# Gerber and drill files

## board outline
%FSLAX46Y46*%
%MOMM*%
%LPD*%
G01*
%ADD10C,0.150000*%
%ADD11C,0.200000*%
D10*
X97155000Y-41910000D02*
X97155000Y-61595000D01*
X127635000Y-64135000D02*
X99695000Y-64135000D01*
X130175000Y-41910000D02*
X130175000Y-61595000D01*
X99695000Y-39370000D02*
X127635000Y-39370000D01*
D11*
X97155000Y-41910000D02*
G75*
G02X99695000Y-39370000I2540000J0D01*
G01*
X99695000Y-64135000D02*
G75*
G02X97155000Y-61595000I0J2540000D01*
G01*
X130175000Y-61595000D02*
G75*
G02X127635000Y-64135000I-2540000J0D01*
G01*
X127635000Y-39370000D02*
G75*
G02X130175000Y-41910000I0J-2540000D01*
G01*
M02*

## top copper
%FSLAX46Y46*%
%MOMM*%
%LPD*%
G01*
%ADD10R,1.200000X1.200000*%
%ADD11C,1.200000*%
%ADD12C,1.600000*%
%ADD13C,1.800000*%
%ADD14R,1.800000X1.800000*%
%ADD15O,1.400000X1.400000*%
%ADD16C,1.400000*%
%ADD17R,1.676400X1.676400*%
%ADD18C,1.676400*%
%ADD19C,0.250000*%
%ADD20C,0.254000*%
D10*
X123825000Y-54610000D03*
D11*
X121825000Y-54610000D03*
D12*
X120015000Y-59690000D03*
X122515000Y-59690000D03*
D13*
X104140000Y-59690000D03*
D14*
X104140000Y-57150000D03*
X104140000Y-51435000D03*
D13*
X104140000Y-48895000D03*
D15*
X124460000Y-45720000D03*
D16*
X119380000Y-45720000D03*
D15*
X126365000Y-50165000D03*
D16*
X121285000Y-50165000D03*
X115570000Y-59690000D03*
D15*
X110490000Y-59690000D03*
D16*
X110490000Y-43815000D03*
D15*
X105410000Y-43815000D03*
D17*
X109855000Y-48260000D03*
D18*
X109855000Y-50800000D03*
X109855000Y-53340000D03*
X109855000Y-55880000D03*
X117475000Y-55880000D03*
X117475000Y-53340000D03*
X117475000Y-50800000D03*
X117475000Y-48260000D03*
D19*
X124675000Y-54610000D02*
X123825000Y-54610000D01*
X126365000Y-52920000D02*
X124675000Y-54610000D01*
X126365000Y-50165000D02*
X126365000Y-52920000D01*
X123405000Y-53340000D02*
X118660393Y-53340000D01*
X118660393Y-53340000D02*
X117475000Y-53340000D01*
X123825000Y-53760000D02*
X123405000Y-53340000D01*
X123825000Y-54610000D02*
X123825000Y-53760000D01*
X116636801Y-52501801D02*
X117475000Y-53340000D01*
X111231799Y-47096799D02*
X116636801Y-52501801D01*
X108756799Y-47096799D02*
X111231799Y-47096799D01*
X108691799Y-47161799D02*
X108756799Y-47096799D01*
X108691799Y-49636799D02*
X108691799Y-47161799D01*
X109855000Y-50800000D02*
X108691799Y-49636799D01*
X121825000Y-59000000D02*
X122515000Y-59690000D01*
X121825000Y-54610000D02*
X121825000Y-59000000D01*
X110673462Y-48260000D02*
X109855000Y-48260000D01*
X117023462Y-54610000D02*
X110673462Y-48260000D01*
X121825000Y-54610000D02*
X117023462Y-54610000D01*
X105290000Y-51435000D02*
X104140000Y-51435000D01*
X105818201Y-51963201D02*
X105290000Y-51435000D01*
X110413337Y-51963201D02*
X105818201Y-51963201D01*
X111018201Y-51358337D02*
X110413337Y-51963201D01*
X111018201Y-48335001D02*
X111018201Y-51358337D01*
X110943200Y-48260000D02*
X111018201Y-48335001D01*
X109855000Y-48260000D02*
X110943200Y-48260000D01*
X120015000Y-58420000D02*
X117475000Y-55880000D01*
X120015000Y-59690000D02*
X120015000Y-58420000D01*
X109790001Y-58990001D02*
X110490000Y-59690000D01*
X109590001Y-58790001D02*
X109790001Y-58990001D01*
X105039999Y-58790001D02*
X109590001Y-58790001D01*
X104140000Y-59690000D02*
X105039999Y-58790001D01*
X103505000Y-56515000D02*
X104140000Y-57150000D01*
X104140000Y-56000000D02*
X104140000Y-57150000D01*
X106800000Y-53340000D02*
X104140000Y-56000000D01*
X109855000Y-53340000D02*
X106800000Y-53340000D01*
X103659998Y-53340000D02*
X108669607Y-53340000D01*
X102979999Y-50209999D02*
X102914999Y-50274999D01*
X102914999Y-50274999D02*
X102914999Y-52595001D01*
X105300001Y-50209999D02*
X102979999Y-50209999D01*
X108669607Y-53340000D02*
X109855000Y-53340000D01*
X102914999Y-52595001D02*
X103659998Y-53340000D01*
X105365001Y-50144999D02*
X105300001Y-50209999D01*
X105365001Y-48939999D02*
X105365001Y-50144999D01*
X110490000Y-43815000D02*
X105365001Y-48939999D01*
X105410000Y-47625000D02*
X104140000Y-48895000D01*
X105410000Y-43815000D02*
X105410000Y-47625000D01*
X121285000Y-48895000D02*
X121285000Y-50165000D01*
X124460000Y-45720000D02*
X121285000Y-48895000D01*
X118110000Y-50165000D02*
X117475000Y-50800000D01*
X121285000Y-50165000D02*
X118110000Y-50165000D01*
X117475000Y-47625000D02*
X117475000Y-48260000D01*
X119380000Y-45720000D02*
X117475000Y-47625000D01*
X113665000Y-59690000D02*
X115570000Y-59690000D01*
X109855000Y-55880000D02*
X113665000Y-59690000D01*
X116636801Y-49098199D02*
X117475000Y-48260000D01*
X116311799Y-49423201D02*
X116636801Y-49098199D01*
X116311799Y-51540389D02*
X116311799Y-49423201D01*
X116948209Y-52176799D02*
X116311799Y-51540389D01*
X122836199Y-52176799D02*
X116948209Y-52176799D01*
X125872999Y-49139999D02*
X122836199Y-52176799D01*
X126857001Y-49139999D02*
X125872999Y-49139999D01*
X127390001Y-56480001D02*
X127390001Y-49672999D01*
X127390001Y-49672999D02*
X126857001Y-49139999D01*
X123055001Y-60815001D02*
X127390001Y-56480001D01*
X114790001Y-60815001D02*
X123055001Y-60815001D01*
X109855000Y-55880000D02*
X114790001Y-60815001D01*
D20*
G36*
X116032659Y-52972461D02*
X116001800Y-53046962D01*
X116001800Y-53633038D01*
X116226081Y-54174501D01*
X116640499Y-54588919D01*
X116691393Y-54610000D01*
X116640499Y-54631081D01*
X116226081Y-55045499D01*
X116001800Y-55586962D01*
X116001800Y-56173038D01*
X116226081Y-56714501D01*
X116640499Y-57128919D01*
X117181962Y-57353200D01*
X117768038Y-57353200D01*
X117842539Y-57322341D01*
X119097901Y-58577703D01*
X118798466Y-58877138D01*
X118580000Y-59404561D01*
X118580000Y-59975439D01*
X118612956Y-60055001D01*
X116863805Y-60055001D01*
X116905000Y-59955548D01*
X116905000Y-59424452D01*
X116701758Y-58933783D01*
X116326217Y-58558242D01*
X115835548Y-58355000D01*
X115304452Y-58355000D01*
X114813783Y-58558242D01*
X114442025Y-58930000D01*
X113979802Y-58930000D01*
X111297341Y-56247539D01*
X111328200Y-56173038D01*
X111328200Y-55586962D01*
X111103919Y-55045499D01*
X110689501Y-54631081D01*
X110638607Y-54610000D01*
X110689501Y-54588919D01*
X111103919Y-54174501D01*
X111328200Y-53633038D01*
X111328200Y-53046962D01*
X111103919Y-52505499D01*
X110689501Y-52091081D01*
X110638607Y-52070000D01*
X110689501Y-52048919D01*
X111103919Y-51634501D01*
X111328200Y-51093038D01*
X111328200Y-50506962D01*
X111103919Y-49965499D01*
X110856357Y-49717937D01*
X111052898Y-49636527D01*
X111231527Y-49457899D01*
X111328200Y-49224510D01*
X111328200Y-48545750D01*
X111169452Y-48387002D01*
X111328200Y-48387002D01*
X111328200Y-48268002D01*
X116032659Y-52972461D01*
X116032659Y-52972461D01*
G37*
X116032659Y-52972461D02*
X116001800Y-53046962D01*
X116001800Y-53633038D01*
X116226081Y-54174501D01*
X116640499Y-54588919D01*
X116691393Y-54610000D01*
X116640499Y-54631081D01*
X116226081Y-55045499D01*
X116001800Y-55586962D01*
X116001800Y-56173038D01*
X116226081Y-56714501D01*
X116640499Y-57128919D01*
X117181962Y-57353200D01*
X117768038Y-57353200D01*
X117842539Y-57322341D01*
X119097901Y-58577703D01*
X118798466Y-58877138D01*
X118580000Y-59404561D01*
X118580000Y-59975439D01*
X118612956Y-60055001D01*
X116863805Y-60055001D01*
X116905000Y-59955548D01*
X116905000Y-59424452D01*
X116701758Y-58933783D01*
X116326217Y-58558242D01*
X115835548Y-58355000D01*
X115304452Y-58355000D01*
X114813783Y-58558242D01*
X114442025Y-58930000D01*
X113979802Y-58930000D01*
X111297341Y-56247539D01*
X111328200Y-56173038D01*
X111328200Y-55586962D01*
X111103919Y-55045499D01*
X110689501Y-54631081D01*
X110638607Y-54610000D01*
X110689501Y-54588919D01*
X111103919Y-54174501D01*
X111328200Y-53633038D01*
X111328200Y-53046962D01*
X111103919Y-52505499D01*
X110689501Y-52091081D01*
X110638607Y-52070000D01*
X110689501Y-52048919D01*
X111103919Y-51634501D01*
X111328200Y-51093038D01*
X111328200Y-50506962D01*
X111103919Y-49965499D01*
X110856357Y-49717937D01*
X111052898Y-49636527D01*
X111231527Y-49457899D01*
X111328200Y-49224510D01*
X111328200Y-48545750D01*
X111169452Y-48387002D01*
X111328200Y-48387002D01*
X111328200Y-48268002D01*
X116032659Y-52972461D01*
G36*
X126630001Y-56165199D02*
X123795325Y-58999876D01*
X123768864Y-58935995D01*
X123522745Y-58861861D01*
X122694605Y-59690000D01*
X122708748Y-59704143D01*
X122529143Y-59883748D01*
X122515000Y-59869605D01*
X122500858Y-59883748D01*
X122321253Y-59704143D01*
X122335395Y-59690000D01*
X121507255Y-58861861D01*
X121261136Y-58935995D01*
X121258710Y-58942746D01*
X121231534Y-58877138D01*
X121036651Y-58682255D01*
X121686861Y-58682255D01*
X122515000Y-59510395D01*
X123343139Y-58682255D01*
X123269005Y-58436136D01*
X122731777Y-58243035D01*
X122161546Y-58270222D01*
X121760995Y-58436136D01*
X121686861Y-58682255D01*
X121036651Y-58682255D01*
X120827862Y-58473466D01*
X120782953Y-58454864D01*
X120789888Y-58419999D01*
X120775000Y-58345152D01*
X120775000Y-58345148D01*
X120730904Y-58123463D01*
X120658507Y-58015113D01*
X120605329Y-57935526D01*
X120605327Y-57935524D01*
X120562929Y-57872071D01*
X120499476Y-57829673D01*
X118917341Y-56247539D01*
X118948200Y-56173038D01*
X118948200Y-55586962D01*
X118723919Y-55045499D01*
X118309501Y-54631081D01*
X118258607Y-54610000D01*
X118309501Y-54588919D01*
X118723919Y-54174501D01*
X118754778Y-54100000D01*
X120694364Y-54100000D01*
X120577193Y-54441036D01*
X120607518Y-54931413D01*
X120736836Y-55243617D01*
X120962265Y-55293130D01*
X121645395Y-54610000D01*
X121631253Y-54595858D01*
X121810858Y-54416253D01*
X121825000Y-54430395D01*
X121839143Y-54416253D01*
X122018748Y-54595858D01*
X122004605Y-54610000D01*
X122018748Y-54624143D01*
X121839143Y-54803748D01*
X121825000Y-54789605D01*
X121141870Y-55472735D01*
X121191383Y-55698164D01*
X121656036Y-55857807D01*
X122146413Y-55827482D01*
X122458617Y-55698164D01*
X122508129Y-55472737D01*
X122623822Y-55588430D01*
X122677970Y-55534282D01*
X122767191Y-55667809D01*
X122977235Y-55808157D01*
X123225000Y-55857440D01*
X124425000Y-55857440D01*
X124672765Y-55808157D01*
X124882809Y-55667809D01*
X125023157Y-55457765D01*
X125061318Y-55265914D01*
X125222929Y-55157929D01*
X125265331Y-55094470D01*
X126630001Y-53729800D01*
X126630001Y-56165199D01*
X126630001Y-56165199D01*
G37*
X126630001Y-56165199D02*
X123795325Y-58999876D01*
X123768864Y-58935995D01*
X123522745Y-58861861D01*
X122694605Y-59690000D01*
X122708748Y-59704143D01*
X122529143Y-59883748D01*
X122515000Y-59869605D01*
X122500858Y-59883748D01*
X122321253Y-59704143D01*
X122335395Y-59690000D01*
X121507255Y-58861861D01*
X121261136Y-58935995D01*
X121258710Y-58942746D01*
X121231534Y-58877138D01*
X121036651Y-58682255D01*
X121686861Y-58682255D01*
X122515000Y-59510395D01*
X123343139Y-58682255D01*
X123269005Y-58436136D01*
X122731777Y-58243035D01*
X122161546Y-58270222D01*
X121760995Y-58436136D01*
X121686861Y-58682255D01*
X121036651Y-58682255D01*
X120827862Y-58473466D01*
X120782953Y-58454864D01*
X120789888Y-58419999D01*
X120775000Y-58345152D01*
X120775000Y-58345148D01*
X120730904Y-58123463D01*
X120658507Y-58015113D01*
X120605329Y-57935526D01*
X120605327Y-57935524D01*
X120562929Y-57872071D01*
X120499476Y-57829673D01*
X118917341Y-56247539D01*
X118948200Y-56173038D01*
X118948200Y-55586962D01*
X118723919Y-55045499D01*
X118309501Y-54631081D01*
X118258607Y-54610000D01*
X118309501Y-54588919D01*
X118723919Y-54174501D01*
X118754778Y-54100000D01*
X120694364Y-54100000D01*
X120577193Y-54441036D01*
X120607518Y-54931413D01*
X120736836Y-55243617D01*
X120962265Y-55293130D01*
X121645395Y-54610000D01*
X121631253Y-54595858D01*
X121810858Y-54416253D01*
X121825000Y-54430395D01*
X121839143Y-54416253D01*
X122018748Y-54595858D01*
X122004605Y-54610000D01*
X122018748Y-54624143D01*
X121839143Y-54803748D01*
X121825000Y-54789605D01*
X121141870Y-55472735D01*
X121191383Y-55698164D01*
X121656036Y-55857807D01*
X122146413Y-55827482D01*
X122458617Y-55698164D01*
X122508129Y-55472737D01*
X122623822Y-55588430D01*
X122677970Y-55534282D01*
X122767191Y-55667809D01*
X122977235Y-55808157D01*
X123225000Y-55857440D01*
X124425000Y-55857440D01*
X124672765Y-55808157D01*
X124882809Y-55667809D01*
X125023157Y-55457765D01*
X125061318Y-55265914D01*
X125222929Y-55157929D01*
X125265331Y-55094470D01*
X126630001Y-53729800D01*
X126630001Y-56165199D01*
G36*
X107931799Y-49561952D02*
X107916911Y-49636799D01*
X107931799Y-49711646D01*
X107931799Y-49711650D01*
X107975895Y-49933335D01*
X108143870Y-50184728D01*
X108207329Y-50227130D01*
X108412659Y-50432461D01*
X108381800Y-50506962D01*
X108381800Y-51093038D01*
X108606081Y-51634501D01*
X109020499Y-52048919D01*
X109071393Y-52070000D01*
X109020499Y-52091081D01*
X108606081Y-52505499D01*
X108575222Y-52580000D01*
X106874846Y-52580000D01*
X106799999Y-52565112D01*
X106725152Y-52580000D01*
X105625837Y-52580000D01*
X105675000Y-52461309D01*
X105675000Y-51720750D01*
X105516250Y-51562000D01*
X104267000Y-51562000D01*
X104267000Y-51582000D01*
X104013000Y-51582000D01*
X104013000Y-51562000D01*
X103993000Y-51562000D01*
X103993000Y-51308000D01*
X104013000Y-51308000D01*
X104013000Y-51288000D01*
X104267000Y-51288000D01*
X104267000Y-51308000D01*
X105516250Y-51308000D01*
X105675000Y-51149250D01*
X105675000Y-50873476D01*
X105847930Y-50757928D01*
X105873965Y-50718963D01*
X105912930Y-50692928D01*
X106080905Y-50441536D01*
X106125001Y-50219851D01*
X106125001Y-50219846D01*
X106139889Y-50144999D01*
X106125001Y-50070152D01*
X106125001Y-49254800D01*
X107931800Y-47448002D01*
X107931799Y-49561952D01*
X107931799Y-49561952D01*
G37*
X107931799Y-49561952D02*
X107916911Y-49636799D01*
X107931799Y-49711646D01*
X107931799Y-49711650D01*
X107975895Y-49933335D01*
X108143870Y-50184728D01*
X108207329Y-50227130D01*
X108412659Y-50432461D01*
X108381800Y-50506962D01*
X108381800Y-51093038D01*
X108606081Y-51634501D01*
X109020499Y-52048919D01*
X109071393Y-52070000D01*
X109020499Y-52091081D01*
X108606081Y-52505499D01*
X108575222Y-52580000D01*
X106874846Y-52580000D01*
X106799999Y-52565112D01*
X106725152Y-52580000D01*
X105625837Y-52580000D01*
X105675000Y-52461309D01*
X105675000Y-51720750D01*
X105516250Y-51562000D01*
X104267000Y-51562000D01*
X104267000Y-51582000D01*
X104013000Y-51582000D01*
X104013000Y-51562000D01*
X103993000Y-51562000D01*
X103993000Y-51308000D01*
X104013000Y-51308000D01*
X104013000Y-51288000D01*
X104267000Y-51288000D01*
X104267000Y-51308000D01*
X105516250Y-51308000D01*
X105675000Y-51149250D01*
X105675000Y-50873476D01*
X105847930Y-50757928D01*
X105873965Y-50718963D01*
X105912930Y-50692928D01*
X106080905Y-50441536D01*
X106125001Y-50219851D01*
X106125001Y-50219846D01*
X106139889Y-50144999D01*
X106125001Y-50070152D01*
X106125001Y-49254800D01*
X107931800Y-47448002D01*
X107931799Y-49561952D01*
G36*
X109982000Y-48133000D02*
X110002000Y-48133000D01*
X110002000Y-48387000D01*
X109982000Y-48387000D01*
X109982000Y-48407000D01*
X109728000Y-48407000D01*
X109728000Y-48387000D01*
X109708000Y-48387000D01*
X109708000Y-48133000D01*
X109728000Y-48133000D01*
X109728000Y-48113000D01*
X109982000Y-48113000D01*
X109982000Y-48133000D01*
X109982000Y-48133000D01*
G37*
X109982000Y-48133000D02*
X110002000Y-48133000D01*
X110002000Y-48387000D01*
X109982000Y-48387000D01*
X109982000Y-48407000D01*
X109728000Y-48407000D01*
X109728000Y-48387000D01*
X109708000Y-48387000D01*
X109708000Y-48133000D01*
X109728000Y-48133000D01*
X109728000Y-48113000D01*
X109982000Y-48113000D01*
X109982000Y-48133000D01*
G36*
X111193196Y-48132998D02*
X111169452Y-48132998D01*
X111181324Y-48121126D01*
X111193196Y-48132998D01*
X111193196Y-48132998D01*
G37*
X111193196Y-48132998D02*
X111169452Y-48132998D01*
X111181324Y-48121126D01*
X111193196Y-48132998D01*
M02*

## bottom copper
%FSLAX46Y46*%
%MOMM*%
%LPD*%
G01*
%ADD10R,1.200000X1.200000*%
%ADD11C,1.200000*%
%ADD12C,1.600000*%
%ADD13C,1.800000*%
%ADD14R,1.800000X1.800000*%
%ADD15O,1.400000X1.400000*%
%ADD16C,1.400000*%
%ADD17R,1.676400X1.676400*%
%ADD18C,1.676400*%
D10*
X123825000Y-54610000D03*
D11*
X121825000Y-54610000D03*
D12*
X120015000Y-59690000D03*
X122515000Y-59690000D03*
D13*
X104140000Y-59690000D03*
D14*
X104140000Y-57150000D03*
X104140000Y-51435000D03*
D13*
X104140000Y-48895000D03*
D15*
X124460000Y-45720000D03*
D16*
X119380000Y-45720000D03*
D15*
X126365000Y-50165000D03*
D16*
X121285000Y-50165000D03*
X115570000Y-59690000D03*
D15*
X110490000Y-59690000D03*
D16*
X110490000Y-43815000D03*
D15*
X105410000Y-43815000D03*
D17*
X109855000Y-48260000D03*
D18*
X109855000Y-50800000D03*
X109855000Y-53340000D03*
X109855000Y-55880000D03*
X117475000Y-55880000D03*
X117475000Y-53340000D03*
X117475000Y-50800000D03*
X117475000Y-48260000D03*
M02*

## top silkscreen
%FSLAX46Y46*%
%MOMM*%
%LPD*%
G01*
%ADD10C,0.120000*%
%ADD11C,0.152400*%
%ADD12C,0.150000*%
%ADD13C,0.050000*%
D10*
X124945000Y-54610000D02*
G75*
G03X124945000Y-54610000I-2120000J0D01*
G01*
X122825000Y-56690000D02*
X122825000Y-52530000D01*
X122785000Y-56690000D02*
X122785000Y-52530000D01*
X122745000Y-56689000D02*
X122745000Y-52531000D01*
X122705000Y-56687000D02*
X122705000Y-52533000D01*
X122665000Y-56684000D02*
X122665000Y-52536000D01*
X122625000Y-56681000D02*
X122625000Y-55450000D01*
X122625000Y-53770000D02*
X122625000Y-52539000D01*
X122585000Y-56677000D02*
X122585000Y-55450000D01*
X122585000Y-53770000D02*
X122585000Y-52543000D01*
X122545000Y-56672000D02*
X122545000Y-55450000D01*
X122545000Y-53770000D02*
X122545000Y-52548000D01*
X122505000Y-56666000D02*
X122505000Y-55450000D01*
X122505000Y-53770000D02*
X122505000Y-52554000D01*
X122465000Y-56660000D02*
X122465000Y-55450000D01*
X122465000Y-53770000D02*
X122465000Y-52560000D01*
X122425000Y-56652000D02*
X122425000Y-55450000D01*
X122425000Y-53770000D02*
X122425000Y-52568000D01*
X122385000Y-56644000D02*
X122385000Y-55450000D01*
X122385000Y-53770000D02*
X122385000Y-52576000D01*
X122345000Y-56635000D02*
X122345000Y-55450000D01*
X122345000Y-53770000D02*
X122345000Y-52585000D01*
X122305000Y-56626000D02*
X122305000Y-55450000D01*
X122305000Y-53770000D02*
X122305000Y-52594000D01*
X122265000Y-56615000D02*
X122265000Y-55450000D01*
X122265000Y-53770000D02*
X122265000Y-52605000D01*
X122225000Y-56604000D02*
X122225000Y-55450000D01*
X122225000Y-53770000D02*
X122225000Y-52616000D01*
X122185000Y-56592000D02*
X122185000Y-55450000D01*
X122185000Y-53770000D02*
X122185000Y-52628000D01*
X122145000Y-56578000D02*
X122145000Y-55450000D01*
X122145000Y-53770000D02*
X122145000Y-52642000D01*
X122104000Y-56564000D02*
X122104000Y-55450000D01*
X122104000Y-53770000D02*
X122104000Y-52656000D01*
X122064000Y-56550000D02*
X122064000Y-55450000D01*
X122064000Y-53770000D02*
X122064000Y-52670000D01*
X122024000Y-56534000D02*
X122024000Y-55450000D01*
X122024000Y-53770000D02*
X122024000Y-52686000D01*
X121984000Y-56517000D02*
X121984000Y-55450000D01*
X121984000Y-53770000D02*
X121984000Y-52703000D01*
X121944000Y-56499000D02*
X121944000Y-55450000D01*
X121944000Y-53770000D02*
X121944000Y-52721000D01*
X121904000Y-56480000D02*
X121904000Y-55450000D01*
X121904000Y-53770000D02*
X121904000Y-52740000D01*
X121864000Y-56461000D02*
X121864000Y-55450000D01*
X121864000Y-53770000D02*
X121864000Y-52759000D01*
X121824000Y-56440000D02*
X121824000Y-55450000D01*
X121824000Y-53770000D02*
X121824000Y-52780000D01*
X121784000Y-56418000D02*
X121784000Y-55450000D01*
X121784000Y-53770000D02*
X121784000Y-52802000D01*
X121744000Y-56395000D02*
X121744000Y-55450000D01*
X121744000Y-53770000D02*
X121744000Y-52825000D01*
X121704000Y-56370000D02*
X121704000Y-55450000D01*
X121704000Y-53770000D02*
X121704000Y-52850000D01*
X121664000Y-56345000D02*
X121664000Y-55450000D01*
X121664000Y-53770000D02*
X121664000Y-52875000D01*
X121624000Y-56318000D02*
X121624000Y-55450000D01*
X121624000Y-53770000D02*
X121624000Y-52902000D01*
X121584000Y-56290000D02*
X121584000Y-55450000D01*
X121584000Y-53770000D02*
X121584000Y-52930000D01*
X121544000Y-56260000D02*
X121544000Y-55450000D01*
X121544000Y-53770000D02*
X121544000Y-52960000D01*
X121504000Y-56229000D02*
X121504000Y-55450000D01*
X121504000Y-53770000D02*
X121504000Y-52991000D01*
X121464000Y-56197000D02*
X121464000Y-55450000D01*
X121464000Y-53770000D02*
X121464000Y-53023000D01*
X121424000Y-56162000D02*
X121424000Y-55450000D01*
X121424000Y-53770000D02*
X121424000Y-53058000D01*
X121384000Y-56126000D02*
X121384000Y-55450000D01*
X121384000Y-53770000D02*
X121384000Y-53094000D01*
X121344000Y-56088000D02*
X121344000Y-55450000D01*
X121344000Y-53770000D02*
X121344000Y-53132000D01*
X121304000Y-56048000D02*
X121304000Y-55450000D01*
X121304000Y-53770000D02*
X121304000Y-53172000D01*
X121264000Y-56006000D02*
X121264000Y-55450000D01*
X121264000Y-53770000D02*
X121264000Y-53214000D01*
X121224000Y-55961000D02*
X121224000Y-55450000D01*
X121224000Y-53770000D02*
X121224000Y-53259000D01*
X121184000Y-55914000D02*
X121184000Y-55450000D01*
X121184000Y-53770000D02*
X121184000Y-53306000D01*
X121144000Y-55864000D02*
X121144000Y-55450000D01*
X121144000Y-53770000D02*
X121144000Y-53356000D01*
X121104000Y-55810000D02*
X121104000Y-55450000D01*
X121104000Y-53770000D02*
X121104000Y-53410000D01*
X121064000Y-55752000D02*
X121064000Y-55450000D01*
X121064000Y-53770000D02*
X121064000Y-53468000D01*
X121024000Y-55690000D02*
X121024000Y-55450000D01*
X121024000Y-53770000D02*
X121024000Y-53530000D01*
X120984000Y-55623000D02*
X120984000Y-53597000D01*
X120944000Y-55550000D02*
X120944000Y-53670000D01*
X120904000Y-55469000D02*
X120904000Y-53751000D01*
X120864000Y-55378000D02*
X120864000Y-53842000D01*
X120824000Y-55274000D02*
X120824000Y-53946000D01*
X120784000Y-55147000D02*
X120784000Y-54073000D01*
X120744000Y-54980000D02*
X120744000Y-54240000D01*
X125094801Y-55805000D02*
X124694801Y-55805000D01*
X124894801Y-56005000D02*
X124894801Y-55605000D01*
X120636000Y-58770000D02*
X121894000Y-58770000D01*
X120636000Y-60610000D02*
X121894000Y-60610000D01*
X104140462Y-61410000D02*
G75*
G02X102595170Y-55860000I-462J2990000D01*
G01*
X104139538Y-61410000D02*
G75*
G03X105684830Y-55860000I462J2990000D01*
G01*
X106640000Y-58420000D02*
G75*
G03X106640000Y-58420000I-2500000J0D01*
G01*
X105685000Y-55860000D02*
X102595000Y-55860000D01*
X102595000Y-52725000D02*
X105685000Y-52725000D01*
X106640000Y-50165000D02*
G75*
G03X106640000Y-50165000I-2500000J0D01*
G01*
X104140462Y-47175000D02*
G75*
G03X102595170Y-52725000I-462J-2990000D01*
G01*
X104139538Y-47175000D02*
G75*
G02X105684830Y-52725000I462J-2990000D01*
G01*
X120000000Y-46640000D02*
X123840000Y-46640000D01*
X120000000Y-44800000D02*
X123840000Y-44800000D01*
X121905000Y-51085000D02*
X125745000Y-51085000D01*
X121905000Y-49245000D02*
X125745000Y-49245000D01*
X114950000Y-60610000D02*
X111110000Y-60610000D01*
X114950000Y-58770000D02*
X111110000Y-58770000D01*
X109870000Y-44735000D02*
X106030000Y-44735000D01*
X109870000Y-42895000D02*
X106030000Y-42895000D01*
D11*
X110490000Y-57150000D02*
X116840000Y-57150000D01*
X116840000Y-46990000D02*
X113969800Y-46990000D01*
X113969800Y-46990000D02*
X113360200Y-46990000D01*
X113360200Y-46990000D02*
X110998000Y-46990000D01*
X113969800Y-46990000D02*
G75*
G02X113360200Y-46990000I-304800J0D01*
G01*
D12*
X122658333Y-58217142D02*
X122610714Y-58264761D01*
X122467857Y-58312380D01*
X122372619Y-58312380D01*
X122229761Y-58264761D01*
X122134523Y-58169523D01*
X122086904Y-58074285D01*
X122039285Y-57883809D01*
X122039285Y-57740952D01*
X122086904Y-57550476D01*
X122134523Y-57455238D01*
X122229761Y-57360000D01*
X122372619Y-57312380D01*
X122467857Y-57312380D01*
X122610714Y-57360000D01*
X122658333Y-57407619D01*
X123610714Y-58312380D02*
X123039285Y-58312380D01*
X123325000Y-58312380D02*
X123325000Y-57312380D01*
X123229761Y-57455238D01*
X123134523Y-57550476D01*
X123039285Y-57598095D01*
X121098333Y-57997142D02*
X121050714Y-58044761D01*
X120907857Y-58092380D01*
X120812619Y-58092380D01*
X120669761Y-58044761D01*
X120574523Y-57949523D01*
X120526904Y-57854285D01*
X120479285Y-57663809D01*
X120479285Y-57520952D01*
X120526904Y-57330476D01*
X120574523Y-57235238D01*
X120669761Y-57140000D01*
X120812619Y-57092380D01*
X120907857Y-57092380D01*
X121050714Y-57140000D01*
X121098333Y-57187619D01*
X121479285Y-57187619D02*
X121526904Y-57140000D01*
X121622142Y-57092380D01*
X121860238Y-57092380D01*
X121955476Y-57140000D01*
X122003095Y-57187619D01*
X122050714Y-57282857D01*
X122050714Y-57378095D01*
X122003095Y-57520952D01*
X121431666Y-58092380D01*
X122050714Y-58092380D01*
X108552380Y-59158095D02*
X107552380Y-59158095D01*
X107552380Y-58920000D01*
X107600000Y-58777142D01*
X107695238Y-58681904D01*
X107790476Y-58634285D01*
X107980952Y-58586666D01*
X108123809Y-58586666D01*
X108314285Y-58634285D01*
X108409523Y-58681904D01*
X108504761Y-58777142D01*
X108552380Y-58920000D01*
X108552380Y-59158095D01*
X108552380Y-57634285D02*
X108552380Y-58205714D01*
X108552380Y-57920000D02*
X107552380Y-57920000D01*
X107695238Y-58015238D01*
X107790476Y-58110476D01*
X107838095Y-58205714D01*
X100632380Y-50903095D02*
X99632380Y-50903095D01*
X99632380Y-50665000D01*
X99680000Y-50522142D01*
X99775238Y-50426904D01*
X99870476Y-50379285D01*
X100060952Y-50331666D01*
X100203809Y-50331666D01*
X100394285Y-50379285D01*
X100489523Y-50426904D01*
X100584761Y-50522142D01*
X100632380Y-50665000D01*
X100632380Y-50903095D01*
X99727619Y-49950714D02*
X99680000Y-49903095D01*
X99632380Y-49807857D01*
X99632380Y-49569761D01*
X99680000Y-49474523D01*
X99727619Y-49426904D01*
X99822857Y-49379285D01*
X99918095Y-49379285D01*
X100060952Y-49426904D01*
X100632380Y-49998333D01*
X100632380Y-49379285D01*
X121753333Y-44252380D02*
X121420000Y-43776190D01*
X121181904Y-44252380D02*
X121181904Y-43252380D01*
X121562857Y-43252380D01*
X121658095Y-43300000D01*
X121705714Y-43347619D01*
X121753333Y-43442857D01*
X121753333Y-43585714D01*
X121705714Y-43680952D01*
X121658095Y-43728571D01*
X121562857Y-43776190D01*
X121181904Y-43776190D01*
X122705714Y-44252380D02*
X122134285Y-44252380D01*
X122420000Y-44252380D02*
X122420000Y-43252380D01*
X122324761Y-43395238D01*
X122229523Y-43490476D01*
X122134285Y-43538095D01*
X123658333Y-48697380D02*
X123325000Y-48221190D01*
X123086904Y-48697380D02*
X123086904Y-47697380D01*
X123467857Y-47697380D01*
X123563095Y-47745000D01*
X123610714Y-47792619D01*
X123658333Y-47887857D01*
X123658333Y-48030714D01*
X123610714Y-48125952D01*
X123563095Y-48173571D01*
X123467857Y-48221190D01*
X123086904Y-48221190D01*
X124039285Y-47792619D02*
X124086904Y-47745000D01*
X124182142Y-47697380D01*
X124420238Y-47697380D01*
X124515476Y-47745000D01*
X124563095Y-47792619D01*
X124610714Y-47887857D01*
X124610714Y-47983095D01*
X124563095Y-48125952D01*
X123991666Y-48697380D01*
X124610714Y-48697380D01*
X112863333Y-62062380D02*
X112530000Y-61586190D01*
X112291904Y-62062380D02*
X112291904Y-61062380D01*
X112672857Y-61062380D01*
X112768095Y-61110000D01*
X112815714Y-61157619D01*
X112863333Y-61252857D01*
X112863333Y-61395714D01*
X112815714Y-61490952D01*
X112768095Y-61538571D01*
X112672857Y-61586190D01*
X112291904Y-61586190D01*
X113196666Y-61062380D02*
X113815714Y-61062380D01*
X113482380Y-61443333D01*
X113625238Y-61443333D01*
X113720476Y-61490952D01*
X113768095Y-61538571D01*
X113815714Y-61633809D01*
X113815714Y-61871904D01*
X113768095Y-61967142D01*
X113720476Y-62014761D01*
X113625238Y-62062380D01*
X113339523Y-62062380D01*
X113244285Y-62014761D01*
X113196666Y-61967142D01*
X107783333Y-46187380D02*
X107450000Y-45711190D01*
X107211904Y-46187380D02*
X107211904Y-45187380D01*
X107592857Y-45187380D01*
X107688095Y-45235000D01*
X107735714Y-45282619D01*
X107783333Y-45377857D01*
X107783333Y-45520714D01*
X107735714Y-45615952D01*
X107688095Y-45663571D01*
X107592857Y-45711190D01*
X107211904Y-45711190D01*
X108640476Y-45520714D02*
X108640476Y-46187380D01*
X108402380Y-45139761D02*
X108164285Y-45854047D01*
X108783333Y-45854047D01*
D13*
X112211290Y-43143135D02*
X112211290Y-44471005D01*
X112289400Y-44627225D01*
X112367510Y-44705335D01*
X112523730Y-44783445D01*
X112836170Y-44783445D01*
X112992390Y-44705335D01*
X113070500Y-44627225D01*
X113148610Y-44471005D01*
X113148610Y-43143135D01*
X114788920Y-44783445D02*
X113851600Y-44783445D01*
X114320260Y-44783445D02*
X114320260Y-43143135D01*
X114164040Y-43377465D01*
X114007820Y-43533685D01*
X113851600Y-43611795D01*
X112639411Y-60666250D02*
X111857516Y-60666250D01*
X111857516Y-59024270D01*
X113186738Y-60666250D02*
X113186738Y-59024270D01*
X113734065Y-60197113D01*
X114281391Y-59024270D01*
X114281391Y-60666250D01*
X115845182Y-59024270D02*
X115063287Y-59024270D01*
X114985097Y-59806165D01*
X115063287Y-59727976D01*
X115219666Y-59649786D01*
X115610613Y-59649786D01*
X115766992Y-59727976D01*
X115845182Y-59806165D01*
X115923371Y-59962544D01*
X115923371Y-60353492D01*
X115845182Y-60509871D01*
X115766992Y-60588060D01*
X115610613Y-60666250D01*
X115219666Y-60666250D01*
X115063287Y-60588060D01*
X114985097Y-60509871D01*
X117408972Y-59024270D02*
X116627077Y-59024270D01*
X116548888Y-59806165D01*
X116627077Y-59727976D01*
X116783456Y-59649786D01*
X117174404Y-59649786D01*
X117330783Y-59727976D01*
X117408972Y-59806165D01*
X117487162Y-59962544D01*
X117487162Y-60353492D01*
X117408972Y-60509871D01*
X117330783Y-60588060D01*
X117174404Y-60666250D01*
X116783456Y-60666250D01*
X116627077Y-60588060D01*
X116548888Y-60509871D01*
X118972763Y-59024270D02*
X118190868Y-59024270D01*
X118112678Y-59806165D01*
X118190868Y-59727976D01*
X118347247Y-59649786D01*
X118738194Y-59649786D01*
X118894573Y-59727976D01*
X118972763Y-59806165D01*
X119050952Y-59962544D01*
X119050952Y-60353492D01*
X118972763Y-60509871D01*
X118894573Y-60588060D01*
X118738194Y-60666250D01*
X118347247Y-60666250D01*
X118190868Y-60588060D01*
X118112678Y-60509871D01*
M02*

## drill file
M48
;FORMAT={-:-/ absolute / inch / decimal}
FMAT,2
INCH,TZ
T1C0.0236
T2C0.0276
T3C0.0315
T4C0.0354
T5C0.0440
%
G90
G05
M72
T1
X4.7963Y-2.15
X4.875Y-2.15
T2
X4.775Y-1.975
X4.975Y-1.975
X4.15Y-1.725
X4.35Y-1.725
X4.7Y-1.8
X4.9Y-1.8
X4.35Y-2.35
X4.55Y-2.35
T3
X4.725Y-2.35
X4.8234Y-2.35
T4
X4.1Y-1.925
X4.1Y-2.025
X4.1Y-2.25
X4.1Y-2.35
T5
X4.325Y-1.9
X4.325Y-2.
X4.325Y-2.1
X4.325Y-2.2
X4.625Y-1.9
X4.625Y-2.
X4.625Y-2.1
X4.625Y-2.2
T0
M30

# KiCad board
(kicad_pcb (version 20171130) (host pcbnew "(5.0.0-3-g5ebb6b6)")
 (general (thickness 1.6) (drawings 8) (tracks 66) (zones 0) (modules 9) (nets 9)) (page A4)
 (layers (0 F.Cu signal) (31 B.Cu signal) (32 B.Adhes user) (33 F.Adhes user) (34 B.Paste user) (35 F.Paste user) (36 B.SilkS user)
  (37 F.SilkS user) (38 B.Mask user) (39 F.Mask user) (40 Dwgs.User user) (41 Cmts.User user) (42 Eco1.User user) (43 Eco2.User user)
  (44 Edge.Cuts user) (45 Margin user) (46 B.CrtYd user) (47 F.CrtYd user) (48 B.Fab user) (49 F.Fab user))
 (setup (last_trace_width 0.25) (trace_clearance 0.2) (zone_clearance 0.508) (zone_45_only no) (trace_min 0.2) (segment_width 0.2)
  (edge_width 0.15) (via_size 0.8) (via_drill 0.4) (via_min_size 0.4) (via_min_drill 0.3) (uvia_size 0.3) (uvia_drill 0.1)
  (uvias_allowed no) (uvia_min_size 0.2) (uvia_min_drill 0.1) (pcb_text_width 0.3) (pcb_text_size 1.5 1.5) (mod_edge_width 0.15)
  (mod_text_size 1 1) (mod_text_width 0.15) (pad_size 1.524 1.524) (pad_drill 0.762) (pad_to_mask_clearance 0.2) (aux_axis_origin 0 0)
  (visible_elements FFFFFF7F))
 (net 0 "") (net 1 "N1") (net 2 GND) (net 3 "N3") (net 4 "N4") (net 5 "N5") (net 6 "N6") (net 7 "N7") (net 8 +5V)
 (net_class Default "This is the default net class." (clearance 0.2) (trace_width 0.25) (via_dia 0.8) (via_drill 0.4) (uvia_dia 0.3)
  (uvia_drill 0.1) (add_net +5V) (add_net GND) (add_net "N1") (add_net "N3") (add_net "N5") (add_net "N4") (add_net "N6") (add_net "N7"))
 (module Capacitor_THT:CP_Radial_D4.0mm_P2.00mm (layer F.Cu) (at 123.825 54.61 180)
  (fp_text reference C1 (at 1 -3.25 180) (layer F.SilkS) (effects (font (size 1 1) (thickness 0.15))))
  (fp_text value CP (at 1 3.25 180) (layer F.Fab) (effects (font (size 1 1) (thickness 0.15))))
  (fp_circle (center 1 0) (end 3.12 0) (layer F.SilkS) (width 0.12))
  (fp_line (start 1 -2.08) (end 1 2.08) (layer F.SilkS) (width 0.12))
  (fp_line (start 1.04 -2.08) (end 1.04 2.08) (layer F.SilkS) (width 0.12))
  (fp_line (start 1.08 -2.079) (end 1.08 2.079) (layer F.SilkS) (width 0.12))
  (fp_line (start 1.12 -2.077) (end 1.12 2.077) (layer F.SilkS) (width 0.12))
  (fp_line (start 1.16 -2.074) (end 1.16 2.074) (layer F.SilkS) (width 0.12))
  (fp_line (start 1.2 -2.071) (end 1.2 -0.84) (layer F.SilkS) (width 0.12))
  (fp_line (start 1.2 0.84) (end 1.2 2.071) (layer F.SilkS) (width 0.12))
  (fp_line (start 1.24 -2.067) (end 1.24 -0.84) (layer F.SilkS) (width 0.12))
  (fp_line (start 1.24 0.84) (end 1.24 2.067) (layer F.SilkS) (width 0.12))
  (fp_line (start 1.28 -2.062) (end 1.28 -0.84) (layer F.SilkS) (width 0.12))
  (fp_line (start 1.28 0.84) (end 1.28 2.062) (layer F.SilkS) (width 0.12))
  (fp_line (start 1.32 -2.056) (end 1.32 -0.84) (layer F.SilkS) (width 0.12))
  (fp_line (start 1.32 0.84) (end 1.32 2.056) (layer F.SilkS) (width 0.12))
  (fp_line (start 1.36 -2.05) (end 1.36 -0.84) (layer F.SilkS) (width 0.12))
  (fp_line (start 1.36 0.84) (end 1.36 2.05) (layer F.SilkS) (width 0.12))
  (fp_line (start 1.4 -2.042) (end 1.4 -0.84) (layer F.SilkS) (width 0.12))
  (fp_line (start 1.4 0.84) (end 1.4 2.042) (layer F.SilkS) (width 0.12))
  (fp_line (start 1.44 -2.034) (end 1.44 -0.84) (layer F.SilkS) (width 0.12))
  (fp_line (start 1.44 0.84) (end 1.44 2.034) (layer F.SilkS) (width 0.12))
  (fp_line (start 1.48 -2.025) (end 1.48 -0.84) (layer F.SilkS) (width 0.12))
  (fp_line (start 1.48 0.84) (end 1.48 2.025) (layer F.SilkS) (width 0.12))
  (fp_line (start 1.52 -2.016) (end 1.52 -0.84) (layer F.SilkS) (width 0.12))
  (fp_line (start 1.52 0.84) (end 1.52 2.016) (layer F.SilkS) (width 0.12))
  (fp_line (start 1.56 -2.005) (end 1.56 -0.84) (layer F.SilkS) (width 0.12))
  (fp_line (start 1.56 0.84) (end 1.56 2.005) (layer F.SilkS) (width 0.12))
  (fp_line (start 1.6 -1.994) (end 1.6 -0.84) (layer F.SilkS) (width 0.12))
  (fp_line (start 1.6 0.84) (end 1.6 1.994) (layer F.SilkS) (width 0.12))
  (fp_line (start 1.64 -1.982) (end 1.64 -0.84) (layer F.SilkS) (width 0.12))
  (fp_line (start 1.64 0.84) (end 1.64 1.982) (layer F.SilkS) (width 0.12))
  (fp_line (start 1.68 -1.968) (end 1.68 -0.84) (layer F.SilkS) (width 0.12))
  (fp_line (start 1.68 0.84) (end 1.68 1.968) (layer F.SilkS) (width 0.12))
  (fp_line (start 1.721 -1.954) (end 1.721 -0.84) (layer F.SilkS) (width 0.12))
  (fp_line (start 1.721 0.84) (end 1.721 1.954) (layer F.SilkS) (width 0.12))
  (fp_line (start 1.761 -1.94) (end 1.761 -0.84) (layer F.SilkS) (width 0.12))
  (fp_line (start 1.761 0.84) (end 1.761 1.94) (layer F.SilkS) (width 0.12))
  (fp_line (start 1.801 -1.924) (end 1.801 -0.84) (layer F.SilkS) (width 0.12))
  (fp_line (start 1.801 0.84) (end 1.801 1.924) (layer F.SilkS) (width 0.12))
  (fp_line (start 1.841 -1.907) (end 1.841 -0.84) (layer F.SilkS) (width 0.12))
  (fp_line (start 1.841 0.84) (end 1.841 1.907) (layer F.SilkS) (width 0.12))
  (fp_line (start 1.881 -1.889) (end 1.881 -0.84) (layer F.SilkS) (width 0.12))
  (fp_line (start 1.881 0.84) (end 1.881 1.889) (layer F.SilkS) (width 0.12))
  (fp_line (start 1.921 -1.87) (end 1.921 -0.84) (layer F.SilkS) (width 0.12))
  (fp_line (start 1.921 0.84) (end 1.921 1.87) (layer F.SilkS) (width 0.12))
  (fp_line (start 1.961 -1.851) (end 1.961 -0.84) (layer F.SilkS) (width 0.12))
  (fp_line (start 1.961 0.84) (end 1.961 1.851) (layer F.SilkS) (width 0.12))
  (fp_line (start 2.001 -1.83) (end 2.001 -0.84) (layer F.SilkS) (width 0.12))
  (fp_line (start 2.001 0.84) (end 2.001 1.83) (layer F.SilkS) (width 0.12))
  (fp_line (start 2.041 -1.808) (end 2.041 -0.84) (layer F.SilkS) (width 0.12))
  (fp_line (start 2.041 0.84) (end 2.041 1.808) (layer F.SilkS) (width 0.12))
  (fp_line (start 2.081 -1.785) (end 2.081 -0.84) (layer F.SilkS) (width 0.12))
  (fp_line (start 2.081 0.84) (end 2.081 1.785) (layer F.SilkS) (width 0.12))
  (fp_line (start 2.121 -1.76) (end 2.121 -0.84) (layer F.SilkS) (width 0.12))
  (fp_line (start 2.121 0.84) (end 2.121 1.76) (layer F.SilkS) (width 0.12))
  (fp_line (start 2.161 -1.735) (end 2.161 -0.84) (layer F.SilkS) (width 0.12))
  (fp_line (start 2.161 0.84) (end 2.161 1.735) (layer F.SilkS) (width 0.12))
  (fp_line (start 2.201 -1.708) (end 2.201 -0.84) (layer F.SilkS) (width 0.12))
  (fp_line (start 2.201 0.84) (end 2.201 1.708) (layer F.SilkS) (width 0.12))
  (fp_line (start 2.241 -1.68) (end 2.241 -0.84) (layer F.SilkS) (width 0.12))
  (fp_line (start 2.241 0.84) (end 2.241 1.68) (layer F.SilkS) (width 0.12))
  (fp_line (start 2.281 -1.65) (end 2.281 -0.84) (layer F.SilkS) (width 0.12))
  (fp_line (start 2.281 0.84) (end 2.281 1.65) (layer F.SilkS) (width 0.12))
  (fp_line (start 2.321 -1.619) (end 2.321 -0.84) (layer F.SilkS) (width 0.12))
  (fp_line (start 2.321 0.84) (end 2.321 1.619) (layer F.SilkS) (width 0.12))
  (fp_line (start 2.361 -1.587) (end 2.361 -0.84) (layer F.SilkS) (width 0.12))
  (fp_line (start 2.361 0.84) (end 2.361 1.587) (layer F.SilkS) (width 0.12))
  (fp_line (start 2.401 -1.552) (end 2.401 -0.84) (layer F.SilkS) (width 0.12))
  (fp_line (start 2.401 0.84) (end 2.401 1.552) (layer F.SilkS) (width 0.12))
  (fp_line (start 2.441 -1.516) (end 2.441 -0.84) (layer F.SilkS) (width 0.12))
  (fp_line (start 2.441 0.84) (end 2.441 1.516) (layer F.SilkS) (width 0.12))
  (fp_line (start 2.481 -1.478) (end 2.481 -0.84) (layer F.SilkS) (width 0.12))
  (fp_line (start 2.481 0.84) (end 2.481 1.478) (layer F.SilkS) (width 0.12))
  (fp_line (start 2.521 -1.438) (end 2.521 -0.84) (layer F.SilkS) (width 0.12))
  (fp_line (start 2.521 0.84) (end 2.521 1.438) (layer F.SilkS) (width 0.12))
  (fp_line (start 2.561 -1.396) (end 2.561 -0.84) (layer F.SilkS) (width 0.12))
  (fp_line (start 2.561 0.84) (end 2.561 1.396) (layer F.SilkS) (width 0.12))
  (fp_line (start 2.601 -1.351) (end 2.601 -0.84) (layer F.SilkS) (width 0.12))
  (fp_line (start 2.601 0.84) (end 2.601 1.351) (layer F.SilkS) (width 0.12))
  (fp_line (start 2.641 -1.304) (end 2.641 -0.84) (layer F.SilkS) (width 0.12))
  (fp_line (start 2.641 0.84) (end 2.641 1.304) (layer F.SilkS) (width 0.12))
  (fp_line (start 2.681 -1.254) (end 2.681 -0.84) (layer F.SilkS) (width 0.12))
  (fp_line (start 2.681 0.84) (end 2.681 1.254) (layer F.SilkS) (width 0.12))
  (fp_line (start 2.721 -1.2) (end 2.721 -0.84) (layer F.SilkS) (width 0.12))
  (fp_line (start 2.721 0.84) (end 2.721 1.2) (layer F.SilkS) (width 0.12))
  (fp_line (start 2.761 -1.142) (end 2.761 -0.84) (layer F.SilkS) (width 0.12))
  (fp_line (start 2.761 0.84) (end 2.761 1.142) (layer F.SilkS) (width 0.12))
  (fp_line (start 2.801 -1.08) (end 2.801 -0.84) (layer F.SilkS) (width 0.12))
  (fp_line (start 2.801 0.84) (end 2.801 1.08) (layer F.SilkS) (width 0.12))
  (fp_line (start 2.841 -1.013) (end 2.841 1.013) (layer F.SilkS) (width 0.12))
  (fp_line (start 2.881 -0.94) (end 2.881 0.94) (layer F.SilkS) (width 0.12))
  (fp_line (start 2.921 -0.859) (end 2.921 0.859) (layer F.SilkS) (width 0.12))
  (fp_line (start 2.961 -0.768) (end 2.961 0.768) (layer F.SilkS) (width 0.12))
  (fp_line (start 3.001 -0.664) (end 3.001 0.664) (layer F.SilkS) (width 0.12))
  (fp_line (start 3.041 -0.537) (end 3.041 0.537) (layer F.SilkS) (width 0.12))
  (fp_line (start 3.081 -0.37) (end 3.081 0.37) (layer F.SilkS) (width 0.12))
  (fp_line (start -1.269801 -1.195) (end -0.869801 -1.195) (layer F.SilkS) (width 0.12))
  (fp_line (start -1.069801 -1.395) (end -1.069801 -0.995) (layer F.SilkS) (width 0.12))
  (pad 1 thru_hole rect (at 0 0 180) (size 1.2 1.2) (drill 0.6) (layers *.Cu *.Mask) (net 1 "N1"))
  (pad 2 thru_hole circle (at 2 0 180) (size 1.2 1.2) (drill 0.6) (layers *.Cu *.Mask) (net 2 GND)))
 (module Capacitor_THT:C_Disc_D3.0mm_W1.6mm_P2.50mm (layer F.Cu) (at 120.015 59.69)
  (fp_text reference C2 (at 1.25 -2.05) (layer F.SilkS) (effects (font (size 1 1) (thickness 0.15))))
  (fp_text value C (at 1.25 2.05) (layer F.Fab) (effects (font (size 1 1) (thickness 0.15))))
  (fp_line (start 0.621 -0.92) (end 1.879 -0.92) (layer F.SilkS) (width 0.12))
  (fp_line (start 0.621 0.92) (end 1.879 0.92) (layer F.SilkS) (width 0.12))
  (pad 1 thru_hole circle (at 0 0) (size 1.6 1.6) (drill 0.8) (layers *.Cu *.Mask) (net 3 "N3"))
  (pad 2 thru_hole circle (at 2.5 0) (size 1.6 1.6) (drill 0.8) (layers *.Cu *.Mask) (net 2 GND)))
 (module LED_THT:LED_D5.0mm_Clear (layer F.Cu) (at 104.14 57.15 270)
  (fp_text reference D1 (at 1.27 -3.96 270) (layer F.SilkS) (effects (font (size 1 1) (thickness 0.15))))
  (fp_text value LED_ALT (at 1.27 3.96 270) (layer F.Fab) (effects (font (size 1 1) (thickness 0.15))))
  (fp_arc (start 1.27 0) (end -1.29 1.54483) (angle -148.9) (layer F.SilkS) (width 0.12))
  (fp_arc (start 1.27 0) (end -1.29 -1.54483) (angle 148.9) (layer F.SilkS) (width 0.12))
  (fp_circle (center 1.27 0) (end 3.77 0) (layer F.SilkS) (width 0.12))
  (fp_line (start -1.29 -1.545) (end -1.29 1.545) (layer F.SilkS) (width 0.12))
  (pad 2 thru_hole circle (at 2.54 0 270) (size 1.8 1.8) (drill 0.9) (layers *.Cu *.Mask) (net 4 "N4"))
  (pad 1 thru_hole rect (at 0 0 270) (size 1.8 1.8) (drill 0.9) (layers *.Cu *.Mask) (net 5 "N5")))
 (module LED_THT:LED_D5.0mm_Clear (layer F.Cu) (at 104.14 51.435 90)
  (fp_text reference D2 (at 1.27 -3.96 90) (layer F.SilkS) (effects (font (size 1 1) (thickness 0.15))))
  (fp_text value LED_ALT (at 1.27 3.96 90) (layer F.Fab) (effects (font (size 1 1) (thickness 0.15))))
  (fp_line (start -1.29 -1.545) (end -1.29 1.545) (layer F.SilkS) (width 0.12))
  (fp_circle (center 1.27 0) (end 3.77 0) (layer F.SilkS) (width 0.12))
  (fp_arc (start 1.27 0) (end -1.29 -1.54483) (angle 148.9) (layer F.SilkS) (width 0.12))
  (fp_arc (start 1.27 0) (end -1.29 1.54483) (angle -148.9) (layer F.SilkS) (width 0.12))
  (pad 1 thru_hole rect (at 0 0 90) (size 1.8 1.8) (drill 0.9) (layers *.Cu *.Mask) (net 2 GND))
  (pad 2 thru_hole circle (at 2.54 0 90) (size 1.8 1.8) (drill 0.9) (layers *.Cu *.Mask) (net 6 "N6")))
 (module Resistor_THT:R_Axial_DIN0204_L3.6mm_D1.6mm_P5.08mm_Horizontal (layer F.Cu) (at 119.38 45.72)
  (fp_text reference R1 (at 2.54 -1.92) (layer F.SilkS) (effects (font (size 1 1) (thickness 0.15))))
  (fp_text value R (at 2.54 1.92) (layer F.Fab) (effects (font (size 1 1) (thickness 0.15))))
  (fp_line (start 0.62 0.92) (end 4.46 0.92) (layer F.SilkS) (width 0.12))
  (fp_line (start 0.62 -0.92) (end 4.46 -0.92) (layer F.SilkS) (width 0.12))
  (pad 2 thru_hole oval (at 5.08 0) (size 1.4 1.4) (drill 0.7) (layers *.Cu *.Mask) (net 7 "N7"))
  (pad 1 thru_hole circle (at 0 0) (size 1.4 1.4) (drill 0.7) (layers *.Cu *.Mask) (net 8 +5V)))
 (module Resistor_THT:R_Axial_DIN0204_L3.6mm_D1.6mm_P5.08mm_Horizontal (layer F.Cu) (at 121.285 50.165)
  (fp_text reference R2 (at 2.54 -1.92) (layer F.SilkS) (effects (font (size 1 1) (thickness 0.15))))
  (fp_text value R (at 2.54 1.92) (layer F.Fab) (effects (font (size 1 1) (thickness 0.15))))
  (fp_line (start 0.62 0.92) (end 4.46 0.92) (layer F.SilkS) (width 0.12))
  (fp_line (start 0.62 -0.92) (end 4.46 -0.92) (layer F.SilkS) (width 0.12))
  (pad 2 thru_hole oval (at 5.08 0) (size 1.4 1.4) (drill 0.7) (layers *.Cu *.Mask) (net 1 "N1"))
  (pad 1 thru_hole circle (at 0 0) (size 1.4 1.4) (drill 0.7) (layers *.Cu *.Mask) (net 7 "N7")))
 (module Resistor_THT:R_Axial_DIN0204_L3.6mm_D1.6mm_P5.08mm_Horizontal (layer F.Cu) (at 115.57 59.69 180)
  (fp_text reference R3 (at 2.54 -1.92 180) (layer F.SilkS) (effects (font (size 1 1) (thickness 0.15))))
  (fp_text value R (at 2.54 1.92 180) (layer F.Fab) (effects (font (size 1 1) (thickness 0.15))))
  (fp_line (start 0.62 -0.92) (end 4.46 -0.92) (layer F.SilkS) (width 0.12))
  (fp_line (start 0.62 0.92) (end 4.46 0.92) (layer F.SilkS) (width 0.12))
  (pad 1 thru_hole circle (at 0 0 180) (size 1.4 1.4) (drill 0.7) (layers *.Cu *.Mask) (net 8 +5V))
  (pad 2 thru_hole oval (at 5.08 0 180) (size 1.4 1.4) (drill 0.7) (layers *.Cu *.Mask) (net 4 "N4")))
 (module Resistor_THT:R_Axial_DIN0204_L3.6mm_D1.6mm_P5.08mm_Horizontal (layer F.Cu) (at 110.49 43.815 180)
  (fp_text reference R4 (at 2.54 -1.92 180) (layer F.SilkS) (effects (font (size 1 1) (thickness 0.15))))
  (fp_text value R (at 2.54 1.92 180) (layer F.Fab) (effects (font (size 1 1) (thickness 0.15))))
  (fp_line (start 0.62 -0.92) (end 4.46 -0.92) (layer F.SilkS) (width 0.12))
  (fp_line (start 0.62 0.92) (end 4.46 0.92) (layer F.SilkS) (width 0.12))
  (pad 1 thru_hole circle (at 0 0 180) (size 1.4 1.4) (drill 0.7) (layers *.Cu *.Mask) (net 5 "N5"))
  (pad 2 thru_hole oval (at 5.08 0 180) (size 1.4 1.4) (drill 0.7) (layers *.Cu *.Mask) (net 6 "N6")))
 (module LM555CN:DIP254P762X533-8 (layer F.Cu) (at 117.475 55.88)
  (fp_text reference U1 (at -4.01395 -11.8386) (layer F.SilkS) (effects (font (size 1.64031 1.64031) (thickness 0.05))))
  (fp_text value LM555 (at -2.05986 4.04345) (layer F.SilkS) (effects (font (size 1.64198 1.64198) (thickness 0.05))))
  (fp_line (start -6.985 1.27) (end -0.635 1.27) (layer F.SilkS) (width 0.1524))
  (fp_line (start -0.635 -8.89) (end -3.5052 -8.89) (layer F.SilkS) (width 0.1524))
  (fp_line (start -3.5052 -8.89) (end -4.1148 -8.89) (layer F.SilkS) (width 0.1524))
  (fp_line (start -4.1148 -8.89) (end -6.477 -8.89) (layer F.SilkS) (width 0.1524))
  (fp_arc (start -3.81 -8.89) (end -4.1148 -8.89) (angle -180) (layer F.SilkS) (width 0.1524))
  (pad 1 thru_hole rect (at -7.62 -7.62) (size 1.6764 1.6764) (drill 1.1176) (layers *.Cu *.Mask) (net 2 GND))
  (pad 2 thru_hole circle (at -7.62 -5.08) (size 1.6764 1.6764) (drill 1.1176) (layers *.Cu *.Mask) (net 1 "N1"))
  (pad 3 thru_hole circle (at -7.62 -2.54) (size 1.6764 1.6764) (drill 1.1176) (layers *.Cu *.Mask) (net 5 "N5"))
  (pad 4 thru_hole circle (at -7.62 0) (size 1.6764 1.6764) (drill 1.1176) (layers *.Cu *.Mask) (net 8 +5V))
  (pad 5 thru_hole circle (at 0 0) (size 1.6764 1.6764) (drill 1.1176) (layers *.Cu *.Mask) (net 3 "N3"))
  (pad 6 thru_hole circle (at 0 -2.54) (size 1.6764 1.6764) (drill 1.1176) (layers *.Cu *.Mask) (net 1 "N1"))
  (pad 7 thru_hole circle (at 0 -5.08) (size 1.6764 1.6764) (drill 1.1176) (layers *.Cu *.Mask) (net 7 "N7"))
  (pad 8 thru_hole circle (at 0 -7.62) (size 1.6764 1.6764) (drill 1.1176) (layers *.Cu *.Mask) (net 8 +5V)))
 (gr_line (start 97.155 41.91) (end 97.155 61.595) (layer Edge.Cuts) (width 0.15))
 (gr_line (start 127.635 64.135) (end 99.695 64.135) (layer Edge.Cuts) (width 0.15))
 (gr_line (start 130.175 41.91) (end 130.175 61.595) (layer Edge.Cuts) (width 0.15))
 (gr_line (start 99.695 39.37) (end 127.635 39.37) (layer Edge.Cuts) (width 0.15))
 (gr_arc (start 99.695 41.91) (end 99.695 39.37) (angle -90) (layer Edge.Cuts) (width 0.2))
 (gr_arc (start 99.695 61.595) (end 97.155 61.595) (angle -90) (layer Edge.Cuts) (width 0.2))
 (gr_arc (start 127.635 61.595) (end 127.635 64.135) (angle -90) (layer Edge.Cuts) (width 0.2))
 (gr_arc (start 127.635 41.91) (end 130.175 41.91) (angle -90) (layer Edge.Cuts) (width 0.2))
 (segment (start 124.675 54.61) (end 123.825 54.61) (width 0.25) (layer F.Cu) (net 1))
 (segment (start 126.365 52.92) (end 124.675 54.61) (width 0.25) (layer F.Cu) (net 1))
 (segment (start 126.365 50.165) (end 126.365 52.92) (width 0.25) (layer F.Cu) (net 1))
 (segment (start 123.405 53.34) (end 118.660393 53.34) (width 0.25) (layer F.Cu) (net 1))
 (segment (start 118.660393 53.34) (end 117.475 53.34) (width 0.25) (layer F.Cu) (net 1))
 (segment (start 123.825 53.76) (end 123.405 53.34) (width 0.25) (layer F.Cu) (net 1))
 (segment (start 123.825 54.61) (end 123.825 53.76) (width 0.25) (layer F.Cu) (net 1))
 (segment (start 116.636801 52.501801) (end 117.475 53.34) (width 0.25) (layer F.Cu) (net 1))
 (segment (start 111.231799 47.096799) (end 116.636801 52.501801) (width 0.25) (layer F.Cu) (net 1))
 (segment (start 108.756799 47.096799) (end 111.231799 47.096799) (width 0.25) (layer F.Cu) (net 1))
 (segment (start 108.691799 47.161799) (end 108.756799 47.096799) (width 0.25) (layer F.Cu) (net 1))
 (segment (start 108.691799 49.636799) (end 108.691799 47.161799) (width 0.25) (layer F.Cu) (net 1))
 (segment (start 109.855 50.8) (end 108.691799 49.636799) (width 0.25) (layer F.Cu) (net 1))
 (segment (start 121.825 59) (end 122.515 59.69) (width 0.25) (layer F.Cu) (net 2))
 (segment (start 121.825 54.61) (end 121.825 59) (width 0.25) (layer F.Cu) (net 2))
 (segment (start 110.673462 48.26) (end 109.855 48.26) (width 0.25) (layer F.Cu) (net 2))
 (segment (start 117.023462 54.61) (end 110.673462 48.26) (width 0.25) (layer F.Cu) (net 2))
 (segment (start 121.825 54.61) (end 117.023462 54.61) (width 0.25) (layer F.Cu) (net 2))
 (segment (start 105.29 51.435) (end 104.14 51.435) (width 0.25) (layer F.Cu) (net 2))
 (segment (start 105.818201 51.963201) (end 105.29 51.435) (width 0.25) (layer F.Cu) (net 2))
 (segment (start 110.413337 51.963201) (end 105.818201 51.963201) (width 0.25) (layer F.Cu) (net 2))
 (segment (start 111.018201 51.358337) (end 110.413337 51.963201) (width 0.25) (layer F.Cu) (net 2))
 (segment (start 111.018201 48.335001) (end 111.018201 51.358337) (width 0.25) (layer F.Cu) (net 2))
 (segment (start 110.9432 48.26) (end 111.018201 48.335001) (width 0.25) (layer F.Cu) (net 2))
 (segment (start 109.855 48.26) (end 110.9432 48.26) (width 0.25) (layer F.Cu) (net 2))
 (segment (start 120.015 58.42) (end 117.475 55.88) (width 0.25) (layer F.Cu) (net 3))
 (segment (start 120.015 59.69) (end 120.015 58.42) (width 0.25) (layer F.Cu) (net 3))
 (segment (start 109.790001 58.990001) (end 110.49 59.69) (width 0.25) (layer F.Cu) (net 4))
 (segment (start 109.590001 58.790001) (end 109.790001 58.990001) (width 0.25) (layer F.Cu) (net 4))
 (segment (start 105.039999 58.790001) (end 109.590001 58.790001) (width 0.25) (layer F.Cu) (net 4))
 (segment (start 104.14 59.69) (end 105.039999 58.790001) (width 0.25) (layer F.Cu) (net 4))
 (segment (start 103.505 56.515) (end 104.14 57.15) (width 0.25) (layer F.Cu) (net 5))
 (segment (start 104.14 56) (end 104.14 57.15) (width 0.25) (layer F.Cu) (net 5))
 (segment (start 106.8 53.34) (end 104.14 56) (width 0.25) (layer F.Cu) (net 5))
 (segment (start 109.855 53.34) (end 106.8 53.34) (width 0.25) (layer F.Cu) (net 5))
 (segment (start 103.659998 53.34) (end 108.669607 53.34) (width 0.25) (layer F.Cu) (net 5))
 (segment (start 102.979999 50.209999) (end 102.914999 50.274999) (width 0.25) (layer F.Cu) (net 5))
 (segment (start 102.914999 50.274999) (end 102.914999 52.595001) (width 0.25) (layer F.Cu) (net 5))
 (segment (start 105.300001 50.209999) (end 102.979999 50.209999) (width 0.25) (layer F.Cu) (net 5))
 (segment (start 108.669607 53.34) (end 109.855 53.34) (width 0.25) (layer F.Cu) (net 5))
 (segment (start 102.914999 52.595001) (end 103.659998 53.34) (width 0.25) (layer F.Cu) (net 5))
 (segment (start 105.365001 50.144999) (end 105.300001 50.209999) (width 0.25) (layer F.Cu) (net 5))
 (segment (start 105.365001 48.939999) (end 105.365001 50.144999) (width 0.25) (layer F.Cu) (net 5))
 (segment (start 110.49 43.815) (end 105.365001 48.939999) (width 0.25) (layer F.Cu) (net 5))
 (segment (start 105.41 47.625) (end 104.14 48.895) (width 0.25) (layer F.Cu) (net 6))
 (segment (start 105.41 43.815) (end 105.41 47.625) (width 0.25) (layer F.Cu) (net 6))
 (segment (start 121.285 48.895) (end 121.285 50.165) (width 0.25) (layer F.Cu) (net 7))
 (segment (start 124.46 45.72) (end 121.285 48.895) (width 0.25) (layer F.Cu) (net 7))
 (segment (start 118.11 50.165) (end 117.475 50.8) (width 0.25) (layer F.Cu) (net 7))
 (segment (start 121.285 50.165) (end 118.11 50.165) (width 0.25) (layer F.Cu) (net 7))
 (segment (start 117.475 47.625) (end 117.475 48.26) (width 0.25) (layer F.Cu) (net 8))
 (segment (start 119.38 45.72) (end 117.475 47.625) (width 0.25) (layer F.Cu) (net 8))
 (segment (start 113.665 59.69) (end 115.57 59.69) (width 0.25) (layer F.Cu) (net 8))
 (segment (start 109.855 55.88) (end 113.665 59.69) (width 0.25) (layer F.Cu) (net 8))
 (segment (start 116.636801 49.098199) (end 117.475 48.26) (width 0.25) (layer F.Cu) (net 8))
 (segment (start 116.311799 49.423201) (end 116.636801 49.098199) (width 0.25) (layer F.Cu) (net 8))
 (segment (start 116.311799 51.540389) (end 116.311799 49.423201) (width 0.25) (layer F.Cu) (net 8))
 (segment (start 116.948209 52.176799) (end 116.311799 51.540389) (width 0.25) (layer F.Cu) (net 8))
 (segment (start 122.836199 52.176799) (end 116.948209 52.176799) (width 0.25) (layer F.Cu) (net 8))
 (segment (start 125.872999 49.139999) (end 122.836199 52.176799) (width 0.25) (layer F.Cu) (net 8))
 (segment (start 126.857001 49.139999) (end 125.872999 49.139999) (width 0.25) (layer F.Cu) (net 8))
 (segment (start 127.390001 56.480001) (end 127.390001 49.672999) (width 0.25) (layer F.Cu) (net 8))
 (segment (start 127.390001 49.672999) (end 126.857001 49.139999) (width 0.25) (layer F.Cu) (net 8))
 (segment (start 123.055001 60.815001) (end 127.390001 56.480001) (width 0.25) (layer F.Cu) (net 8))
 (segment (start 114.790001 60.815001) (end 123.055001 60.815001) (width 0.25) (layer F.Cu) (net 8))
 (segment (start 109.855 55.88) (end 114.790001 60.815001) (width 0.25) (layer F.Cu) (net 8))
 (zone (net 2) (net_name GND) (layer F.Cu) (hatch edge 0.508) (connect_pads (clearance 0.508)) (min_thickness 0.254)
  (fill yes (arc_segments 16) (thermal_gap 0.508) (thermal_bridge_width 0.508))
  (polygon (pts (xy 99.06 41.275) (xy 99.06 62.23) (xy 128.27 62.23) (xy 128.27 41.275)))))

